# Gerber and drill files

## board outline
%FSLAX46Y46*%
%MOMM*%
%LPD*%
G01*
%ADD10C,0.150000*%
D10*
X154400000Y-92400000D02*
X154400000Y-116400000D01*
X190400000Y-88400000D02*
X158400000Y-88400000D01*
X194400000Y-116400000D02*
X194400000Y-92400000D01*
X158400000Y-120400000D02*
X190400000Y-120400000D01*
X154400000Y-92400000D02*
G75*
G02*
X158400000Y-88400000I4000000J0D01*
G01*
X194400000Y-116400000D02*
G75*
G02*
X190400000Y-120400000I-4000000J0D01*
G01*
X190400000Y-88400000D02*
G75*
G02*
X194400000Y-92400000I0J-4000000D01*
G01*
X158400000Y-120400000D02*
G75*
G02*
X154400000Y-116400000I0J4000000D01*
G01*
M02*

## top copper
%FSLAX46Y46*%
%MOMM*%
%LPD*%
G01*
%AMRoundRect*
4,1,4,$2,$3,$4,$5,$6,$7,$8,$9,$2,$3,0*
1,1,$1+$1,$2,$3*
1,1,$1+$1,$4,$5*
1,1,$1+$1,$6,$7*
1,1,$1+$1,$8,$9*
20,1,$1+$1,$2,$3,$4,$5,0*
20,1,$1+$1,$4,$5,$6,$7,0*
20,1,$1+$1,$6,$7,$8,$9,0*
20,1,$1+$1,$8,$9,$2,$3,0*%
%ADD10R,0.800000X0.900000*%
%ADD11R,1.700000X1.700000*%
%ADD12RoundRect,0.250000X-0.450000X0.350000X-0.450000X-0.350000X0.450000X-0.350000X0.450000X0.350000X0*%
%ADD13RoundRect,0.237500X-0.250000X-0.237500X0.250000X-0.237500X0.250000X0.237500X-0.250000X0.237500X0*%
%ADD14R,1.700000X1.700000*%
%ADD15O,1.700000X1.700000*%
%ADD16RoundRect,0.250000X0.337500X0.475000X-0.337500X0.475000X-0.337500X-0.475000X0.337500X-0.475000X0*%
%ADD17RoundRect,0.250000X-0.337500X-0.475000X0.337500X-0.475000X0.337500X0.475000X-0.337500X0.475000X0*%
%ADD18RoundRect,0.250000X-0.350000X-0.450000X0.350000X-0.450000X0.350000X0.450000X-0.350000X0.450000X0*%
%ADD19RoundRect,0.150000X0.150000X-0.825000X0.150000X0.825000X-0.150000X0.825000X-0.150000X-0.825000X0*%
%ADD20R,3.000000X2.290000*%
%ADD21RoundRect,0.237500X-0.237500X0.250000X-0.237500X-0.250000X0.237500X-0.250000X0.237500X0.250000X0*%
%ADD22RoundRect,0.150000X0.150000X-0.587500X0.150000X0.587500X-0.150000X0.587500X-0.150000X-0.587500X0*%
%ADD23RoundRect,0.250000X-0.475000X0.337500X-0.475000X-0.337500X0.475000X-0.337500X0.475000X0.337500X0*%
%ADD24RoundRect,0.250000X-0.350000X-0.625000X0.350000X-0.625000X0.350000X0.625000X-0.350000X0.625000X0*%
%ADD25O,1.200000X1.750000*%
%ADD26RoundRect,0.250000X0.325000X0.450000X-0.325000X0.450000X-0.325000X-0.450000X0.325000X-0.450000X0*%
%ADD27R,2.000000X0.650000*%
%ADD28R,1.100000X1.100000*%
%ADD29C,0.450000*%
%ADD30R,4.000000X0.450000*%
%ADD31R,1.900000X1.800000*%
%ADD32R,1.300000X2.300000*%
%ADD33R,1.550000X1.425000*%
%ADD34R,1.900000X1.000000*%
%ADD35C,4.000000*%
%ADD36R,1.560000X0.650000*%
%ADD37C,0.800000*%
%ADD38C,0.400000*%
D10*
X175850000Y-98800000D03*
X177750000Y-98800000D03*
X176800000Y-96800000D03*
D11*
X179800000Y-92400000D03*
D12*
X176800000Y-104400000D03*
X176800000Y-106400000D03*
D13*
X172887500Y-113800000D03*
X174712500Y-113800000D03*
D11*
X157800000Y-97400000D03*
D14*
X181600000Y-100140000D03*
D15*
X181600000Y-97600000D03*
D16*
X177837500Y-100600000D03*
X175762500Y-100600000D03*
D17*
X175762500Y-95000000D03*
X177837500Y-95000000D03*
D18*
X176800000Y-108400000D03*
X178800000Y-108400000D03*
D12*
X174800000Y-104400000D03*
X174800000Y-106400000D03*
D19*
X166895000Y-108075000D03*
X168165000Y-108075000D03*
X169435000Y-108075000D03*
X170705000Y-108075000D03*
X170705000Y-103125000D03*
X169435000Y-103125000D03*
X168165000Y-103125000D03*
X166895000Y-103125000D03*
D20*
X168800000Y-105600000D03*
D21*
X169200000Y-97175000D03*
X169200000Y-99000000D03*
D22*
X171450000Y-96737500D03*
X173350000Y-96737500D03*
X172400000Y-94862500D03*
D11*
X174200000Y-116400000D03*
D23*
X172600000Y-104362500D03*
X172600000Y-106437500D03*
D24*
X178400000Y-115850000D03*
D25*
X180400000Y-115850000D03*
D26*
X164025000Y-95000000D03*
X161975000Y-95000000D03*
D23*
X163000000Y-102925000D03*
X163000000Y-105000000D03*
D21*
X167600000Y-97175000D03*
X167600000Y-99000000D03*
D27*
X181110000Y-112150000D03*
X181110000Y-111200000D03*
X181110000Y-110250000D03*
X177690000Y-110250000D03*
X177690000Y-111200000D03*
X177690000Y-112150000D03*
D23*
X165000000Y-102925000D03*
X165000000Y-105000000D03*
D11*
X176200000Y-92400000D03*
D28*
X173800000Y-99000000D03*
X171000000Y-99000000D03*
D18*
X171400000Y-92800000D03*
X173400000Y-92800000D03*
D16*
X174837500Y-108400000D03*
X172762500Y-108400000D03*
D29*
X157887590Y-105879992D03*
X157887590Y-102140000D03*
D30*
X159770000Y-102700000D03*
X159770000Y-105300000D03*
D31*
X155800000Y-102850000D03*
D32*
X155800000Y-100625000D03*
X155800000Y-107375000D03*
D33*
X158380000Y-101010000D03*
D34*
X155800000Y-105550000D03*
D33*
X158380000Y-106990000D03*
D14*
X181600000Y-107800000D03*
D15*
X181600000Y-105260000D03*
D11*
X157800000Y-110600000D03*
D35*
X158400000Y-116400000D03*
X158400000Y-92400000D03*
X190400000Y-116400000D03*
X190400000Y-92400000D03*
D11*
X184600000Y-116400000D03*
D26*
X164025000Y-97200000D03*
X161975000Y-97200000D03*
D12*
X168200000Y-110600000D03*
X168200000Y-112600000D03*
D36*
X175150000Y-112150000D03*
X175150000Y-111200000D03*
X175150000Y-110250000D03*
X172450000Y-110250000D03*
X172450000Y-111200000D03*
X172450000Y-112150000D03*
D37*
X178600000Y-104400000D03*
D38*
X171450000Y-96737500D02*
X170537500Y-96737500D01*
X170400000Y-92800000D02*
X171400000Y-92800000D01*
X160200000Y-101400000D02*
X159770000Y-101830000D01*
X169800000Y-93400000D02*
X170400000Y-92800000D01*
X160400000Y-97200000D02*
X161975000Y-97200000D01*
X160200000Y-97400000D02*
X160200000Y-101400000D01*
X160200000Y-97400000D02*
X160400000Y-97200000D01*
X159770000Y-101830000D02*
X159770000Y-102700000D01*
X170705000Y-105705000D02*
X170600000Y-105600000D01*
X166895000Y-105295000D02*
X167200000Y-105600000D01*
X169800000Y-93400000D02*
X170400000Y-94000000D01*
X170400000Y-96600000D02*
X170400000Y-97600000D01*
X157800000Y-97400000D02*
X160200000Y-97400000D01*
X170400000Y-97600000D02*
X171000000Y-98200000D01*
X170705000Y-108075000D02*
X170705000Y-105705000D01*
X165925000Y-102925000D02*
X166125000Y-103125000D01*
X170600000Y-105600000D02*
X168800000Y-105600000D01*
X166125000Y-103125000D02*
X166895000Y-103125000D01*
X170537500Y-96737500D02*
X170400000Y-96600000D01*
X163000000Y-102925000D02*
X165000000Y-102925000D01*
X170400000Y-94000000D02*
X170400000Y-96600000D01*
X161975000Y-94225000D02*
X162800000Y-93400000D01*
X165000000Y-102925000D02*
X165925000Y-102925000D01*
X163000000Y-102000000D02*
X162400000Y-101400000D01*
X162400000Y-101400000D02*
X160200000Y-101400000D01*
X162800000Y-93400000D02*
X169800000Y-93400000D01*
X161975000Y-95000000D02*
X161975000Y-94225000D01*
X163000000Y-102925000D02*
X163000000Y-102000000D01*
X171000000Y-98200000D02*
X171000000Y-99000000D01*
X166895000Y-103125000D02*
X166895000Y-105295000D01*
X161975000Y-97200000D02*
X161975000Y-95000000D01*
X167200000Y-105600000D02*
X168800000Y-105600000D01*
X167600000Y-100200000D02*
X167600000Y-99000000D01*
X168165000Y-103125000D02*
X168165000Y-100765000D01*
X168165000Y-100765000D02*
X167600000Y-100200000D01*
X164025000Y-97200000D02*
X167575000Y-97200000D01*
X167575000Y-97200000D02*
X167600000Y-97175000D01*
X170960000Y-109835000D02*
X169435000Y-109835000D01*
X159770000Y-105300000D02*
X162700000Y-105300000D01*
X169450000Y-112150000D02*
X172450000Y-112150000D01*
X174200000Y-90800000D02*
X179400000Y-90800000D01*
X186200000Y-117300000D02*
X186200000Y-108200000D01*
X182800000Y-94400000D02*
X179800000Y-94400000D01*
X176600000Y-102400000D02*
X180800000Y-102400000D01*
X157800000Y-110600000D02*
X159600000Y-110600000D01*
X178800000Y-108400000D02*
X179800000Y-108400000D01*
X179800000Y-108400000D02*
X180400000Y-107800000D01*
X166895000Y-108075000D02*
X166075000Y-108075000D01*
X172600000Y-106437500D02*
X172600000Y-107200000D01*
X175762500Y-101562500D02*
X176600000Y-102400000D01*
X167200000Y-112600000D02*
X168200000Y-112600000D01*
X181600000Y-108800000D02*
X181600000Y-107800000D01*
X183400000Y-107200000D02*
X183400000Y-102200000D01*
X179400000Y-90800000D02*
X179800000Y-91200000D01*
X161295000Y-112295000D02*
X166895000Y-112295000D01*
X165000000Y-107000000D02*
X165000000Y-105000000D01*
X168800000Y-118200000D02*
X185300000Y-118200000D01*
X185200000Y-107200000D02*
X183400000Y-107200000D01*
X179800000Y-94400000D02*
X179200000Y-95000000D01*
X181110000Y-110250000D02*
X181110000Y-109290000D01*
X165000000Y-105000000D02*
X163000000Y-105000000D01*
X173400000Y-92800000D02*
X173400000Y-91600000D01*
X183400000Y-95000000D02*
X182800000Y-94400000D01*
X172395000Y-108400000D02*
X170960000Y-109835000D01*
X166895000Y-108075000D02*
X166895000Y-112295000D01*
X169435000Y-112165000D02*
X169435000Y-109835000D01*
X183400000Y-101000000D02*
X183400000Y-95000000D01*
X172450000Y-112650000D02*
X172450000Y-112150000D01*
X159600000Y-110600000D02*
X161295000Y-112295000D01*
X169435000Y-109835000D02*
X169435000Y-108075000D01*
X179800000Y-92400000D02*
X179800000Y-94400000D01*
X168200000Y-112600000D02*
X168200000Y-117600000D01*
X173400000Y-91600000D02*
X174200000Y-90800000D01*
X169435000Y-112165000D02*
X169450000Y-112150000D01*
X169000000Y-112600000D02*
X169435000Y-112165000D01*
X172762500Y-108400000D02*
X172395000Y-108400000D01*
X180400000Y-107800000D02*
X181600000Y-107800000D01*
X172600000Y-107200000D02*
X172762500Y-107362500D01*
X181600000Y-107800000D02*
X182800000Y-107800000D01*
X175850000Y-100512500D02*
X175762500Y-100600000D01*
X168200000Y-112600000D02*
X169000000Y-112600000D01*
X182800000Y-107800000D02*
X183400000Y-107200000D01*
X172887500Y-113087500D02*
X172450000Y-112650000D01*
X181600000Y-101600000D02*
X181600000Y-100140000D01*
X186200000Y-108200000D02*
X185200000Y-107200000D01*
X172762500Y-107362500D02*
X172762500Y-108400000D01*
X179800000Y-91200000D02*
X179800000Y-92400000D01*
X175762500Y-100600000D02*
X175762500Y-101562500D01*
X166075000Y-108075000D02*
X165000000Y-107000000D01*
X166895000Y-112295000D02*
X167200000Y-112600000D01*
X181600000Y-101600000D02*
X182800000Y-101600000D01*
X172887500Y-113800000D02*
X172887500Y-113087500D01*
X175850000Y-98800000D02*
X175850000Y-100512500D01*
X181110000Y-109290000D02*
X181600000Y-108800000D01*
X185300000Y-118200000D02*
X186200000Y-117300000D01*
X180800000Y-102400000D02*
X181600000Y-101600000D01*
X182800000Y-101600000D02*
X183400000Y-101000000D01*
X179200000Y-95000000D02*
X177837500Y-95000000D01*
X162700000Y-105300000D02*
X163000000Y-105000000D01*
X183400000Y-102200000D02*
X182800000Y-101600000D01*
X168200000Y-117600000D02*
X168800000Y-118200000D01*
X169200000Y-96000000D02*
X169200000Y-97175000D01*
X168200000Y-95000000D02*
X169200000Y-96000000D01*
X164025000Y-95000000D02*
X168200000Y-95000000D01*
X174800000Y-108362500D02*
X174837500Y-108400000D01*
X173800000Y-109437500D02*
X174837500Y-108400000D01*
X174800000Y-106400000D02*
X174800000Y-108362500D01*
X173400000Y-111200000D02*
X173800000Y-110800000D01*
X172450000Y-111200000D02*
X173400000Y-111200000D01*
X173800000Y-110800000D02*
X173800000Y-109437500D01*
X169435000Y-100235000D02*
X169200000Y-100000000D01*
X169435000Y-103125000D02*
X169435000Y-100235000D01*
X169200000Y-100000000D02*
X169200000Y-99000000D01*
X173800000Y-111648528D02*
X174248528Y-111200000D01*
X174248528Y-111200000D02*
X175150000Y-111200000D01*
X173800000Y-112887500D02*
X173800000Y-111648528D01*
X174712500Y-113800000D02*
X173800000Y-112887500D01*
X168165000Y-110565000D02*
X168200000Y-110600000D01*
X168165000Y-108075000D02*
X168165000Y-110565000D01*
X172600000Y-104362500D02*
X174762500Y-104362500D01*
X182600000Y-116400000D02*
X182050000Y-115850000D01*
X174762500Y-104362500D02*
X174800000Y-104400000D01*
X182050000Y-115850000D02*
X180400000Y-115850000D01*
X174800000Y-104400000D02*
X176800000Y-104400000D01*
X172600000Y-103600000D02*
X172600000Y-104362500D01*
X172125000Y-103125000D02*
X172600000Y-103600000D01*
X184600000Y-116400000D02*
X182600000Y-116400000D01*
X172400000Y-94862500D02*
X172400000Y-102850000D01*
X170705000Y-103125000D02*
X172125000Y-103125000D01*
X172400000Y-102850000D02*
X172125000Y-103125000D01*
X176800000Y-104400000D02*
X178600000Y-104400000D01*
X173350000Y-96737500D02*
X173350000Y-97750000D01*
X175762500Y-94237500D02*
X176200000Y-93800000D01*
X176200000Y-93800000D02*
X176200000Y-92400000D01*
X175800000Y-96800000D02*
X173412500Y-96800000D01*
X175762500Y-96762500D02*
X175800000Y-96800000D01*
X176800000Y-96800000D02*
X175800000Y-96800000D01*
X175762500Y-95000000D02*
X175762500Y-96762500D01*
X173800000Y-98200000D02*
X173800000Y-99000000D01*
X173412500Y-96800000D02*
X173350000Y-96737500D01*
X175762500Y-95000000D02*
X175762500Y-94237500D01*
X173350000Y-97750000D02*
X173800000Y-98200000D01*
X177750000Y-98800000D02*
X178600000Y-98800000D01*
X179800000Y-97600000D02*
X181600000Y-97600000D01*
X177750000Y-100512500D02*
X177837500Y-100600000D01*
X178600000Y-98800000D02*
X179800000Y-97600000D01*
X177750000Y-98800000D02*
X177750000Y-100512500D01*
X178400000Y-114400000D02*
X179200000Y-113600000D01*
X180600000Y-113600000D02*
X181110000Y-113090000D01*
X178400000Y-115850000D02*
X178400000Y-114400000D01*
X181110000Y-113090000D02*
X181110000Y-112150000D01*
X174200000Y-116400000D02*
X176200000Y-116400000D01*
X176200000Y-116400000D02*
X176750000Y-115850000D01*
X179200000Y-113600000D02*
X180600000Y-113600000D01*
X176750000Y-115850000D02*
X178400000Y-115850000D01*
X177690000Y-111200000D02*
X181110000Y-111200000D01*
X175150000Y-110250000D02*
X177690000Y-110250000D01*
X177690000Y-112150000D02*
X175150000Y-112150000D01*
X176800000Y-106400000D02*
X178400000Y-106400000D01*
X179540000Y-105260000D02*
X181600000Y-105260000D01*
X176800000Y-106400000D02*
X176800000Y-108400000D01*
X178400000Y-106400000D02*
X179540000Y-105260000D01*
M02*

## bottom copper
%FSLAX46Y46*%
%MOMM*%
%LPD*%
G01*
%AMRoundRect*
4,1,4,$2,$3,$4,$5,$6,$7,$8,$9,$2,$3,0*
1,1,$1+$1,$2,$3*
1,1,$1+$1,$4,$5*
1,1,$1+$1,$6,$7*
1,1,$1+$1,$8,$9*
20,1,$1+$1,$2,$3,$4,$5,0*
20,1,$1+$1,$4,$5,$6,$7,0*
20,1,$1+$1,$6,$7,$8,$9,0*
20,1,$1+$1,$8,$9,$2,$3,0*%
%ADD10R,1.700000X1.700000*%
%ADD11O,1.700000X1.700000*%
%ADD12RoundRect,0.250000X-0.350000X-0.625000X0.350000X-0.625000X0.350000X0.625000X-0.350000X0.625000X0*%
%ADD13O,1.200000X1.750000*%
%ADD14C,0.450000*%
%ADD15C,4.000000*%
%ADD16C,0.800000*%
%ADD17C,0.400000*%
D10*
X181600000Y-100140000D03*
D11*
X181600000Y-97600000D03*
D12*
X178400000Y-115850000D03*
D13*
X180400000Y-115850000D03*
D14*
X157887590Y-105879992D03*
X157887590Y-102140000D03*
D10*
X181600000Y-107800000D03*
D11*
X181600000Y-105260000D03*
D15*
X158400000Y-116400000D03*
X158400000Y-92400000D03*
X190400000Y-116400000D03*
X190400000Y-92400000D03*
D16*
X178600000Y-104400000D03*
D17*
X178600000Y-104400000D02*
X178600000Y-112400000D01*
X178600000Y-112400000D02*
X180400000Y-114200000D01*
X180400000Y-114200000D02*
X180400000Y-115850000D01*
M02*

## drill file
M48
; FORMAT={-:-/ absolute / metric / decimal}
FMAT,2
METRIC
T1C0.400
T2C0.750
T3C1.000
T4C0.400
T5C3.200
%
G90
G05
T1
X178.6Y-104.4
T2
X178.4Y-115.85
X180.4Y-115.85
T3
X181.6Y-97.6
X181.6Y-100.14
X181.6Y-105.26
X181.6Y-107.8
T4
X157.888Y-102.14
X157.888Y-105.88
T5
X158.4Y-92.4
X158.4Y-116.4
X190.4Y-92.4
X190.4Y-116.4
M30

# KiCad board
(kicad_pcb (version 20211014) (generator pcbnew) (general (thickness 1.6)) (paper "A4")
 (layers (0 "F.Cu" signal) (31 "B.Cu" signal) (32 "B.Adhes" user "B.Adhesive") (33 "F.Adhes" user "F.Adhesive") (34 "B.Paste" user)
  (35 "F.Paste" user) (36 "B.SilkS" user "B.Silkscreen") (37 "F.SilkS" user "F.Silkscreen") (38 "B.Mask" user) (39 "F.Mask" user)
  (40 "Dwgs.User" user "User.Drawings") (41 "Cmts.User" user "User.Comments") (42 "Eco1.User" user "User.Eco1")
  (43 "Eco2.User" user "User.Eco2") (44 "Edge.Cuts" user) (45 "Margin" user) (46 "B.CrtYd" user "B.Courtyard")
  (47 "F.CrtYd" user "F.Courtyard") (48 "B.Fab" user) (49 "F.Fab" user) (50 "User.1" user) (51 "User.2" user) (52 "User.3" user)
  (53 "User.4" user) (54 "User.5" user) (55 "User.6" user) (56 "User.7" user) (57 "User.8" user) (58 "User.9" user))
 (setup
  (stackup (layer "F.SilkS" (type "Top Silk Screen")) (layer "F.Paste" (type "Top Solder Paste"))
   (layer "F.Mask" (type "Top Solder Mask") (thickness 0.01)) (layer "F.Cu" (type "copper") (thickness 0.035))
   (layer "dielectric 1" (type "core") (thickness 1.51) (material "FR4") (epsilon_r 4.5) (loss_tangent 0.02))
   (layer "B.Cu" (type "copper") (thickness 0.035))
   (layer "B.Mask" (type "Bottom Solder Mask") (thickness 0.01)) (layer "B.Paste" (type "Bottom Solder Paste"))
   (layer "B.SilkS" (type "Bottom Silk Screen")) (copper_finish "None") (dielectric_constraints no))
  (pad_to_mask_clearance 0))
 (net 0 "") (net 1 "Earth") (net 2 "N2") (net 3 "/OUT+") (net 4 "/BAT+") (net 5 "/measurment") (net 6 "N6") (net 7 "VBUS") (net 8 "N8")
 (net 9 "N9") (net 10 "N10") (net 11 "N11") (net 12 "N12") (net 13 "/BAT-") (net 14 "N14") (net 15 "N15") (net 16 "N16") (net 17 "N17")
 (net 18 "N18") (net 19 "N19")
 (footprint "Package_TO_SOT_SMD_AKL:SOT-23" (layer "F.Cu") (at 176.8 97.8 90)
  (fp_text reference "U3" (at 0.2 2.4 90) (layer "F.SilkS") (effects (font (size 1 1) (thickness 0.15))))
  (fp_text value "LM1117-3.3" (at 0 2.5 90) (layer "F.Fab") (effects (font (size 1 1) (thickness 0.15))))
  (pad "1" smd rect (at -1 -0.95 90) (size 0.9 0.8) (layers "F.Cu" "F.Paste" "F.Mask") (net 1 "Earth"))
  (pad "2" smd rect (at -1 0.95 90) (size 0.9 0.8) (layers "F.Cu" "F.Paste" "F.Mask") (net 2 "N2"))
  (pad "3" smd rect (at 1 0 90) (size 0.9 0.8) (layers "F.Cu" "F.Paste" "F.Mask") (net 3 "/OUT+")))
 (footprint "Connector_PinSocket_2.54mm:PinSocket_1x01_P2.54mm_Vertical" (layer "F.Cu") (at 179.8 92.4)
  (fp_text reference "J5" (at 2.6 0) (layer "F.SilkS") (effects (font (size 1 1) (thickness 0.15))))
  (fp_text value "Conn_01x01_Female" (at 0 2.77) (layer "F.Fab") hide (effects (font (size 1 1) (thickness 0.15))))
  (pad "1" smd rect (at 0 0) (size 1.7 1.7) (layers "F.Cu" "F.Paste" "F.Mask") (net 1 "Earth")))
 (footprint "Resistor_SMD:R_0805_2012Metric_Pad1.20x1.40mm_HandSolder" (layer "F.Cu") (at 176.8 105.4 -90)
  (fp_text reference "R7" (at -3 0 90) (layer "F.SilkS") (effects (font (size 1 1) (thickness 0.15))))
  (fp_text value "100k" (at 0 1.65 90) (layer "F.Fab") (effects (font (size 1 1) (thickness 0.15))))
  (pad "1" smd roundrect (at -1 0 270) (size 1.2 1.4) (layers "F.Cu" "F.Paste" "F.Mask") (roundrect_rratio 0.208333) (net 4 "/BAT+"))
  (pad "2" smd roundrect (at 1 0 270) (size 1.2 1.4) (layers "F.Cu" "F.Paste" "F.Mask") (roundrect_rratio 0.208333) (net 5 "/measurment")))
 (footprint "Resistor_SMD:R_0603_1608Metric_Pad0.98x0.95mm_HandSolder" (layer "F.Cu") (at 173.8 113.8)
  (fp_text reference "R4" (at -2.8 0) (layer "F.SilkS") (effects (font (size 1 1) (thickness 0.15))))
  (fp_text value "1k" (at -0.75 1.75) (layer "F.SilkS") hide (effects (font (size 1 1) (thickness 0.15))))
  (pad "1" smd roundrect (at -0.9125 0) (size 0.975 0.95) (layers "F.Cu" "F.Paste" "F.Mask") (roundrect_rratio 0.25) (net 1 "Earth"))
  (pad "2" smd roundrect (at 0.9125 0) (size 0.975 0.95) (layers "F.Cu" "F.Paste" "F.Mask") (roundrect_rratio 0.25) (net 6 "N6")))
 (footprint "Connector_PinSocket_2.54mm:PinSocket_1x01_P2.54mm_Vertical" (layer "F.Cu") (at 157.8 97.4)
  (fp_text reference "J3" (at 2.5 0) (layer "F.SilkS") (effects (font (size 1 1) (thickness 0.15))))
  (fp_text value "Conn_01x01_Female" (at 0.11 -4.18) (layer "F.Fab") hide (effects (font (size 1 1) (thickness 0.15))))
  (pad "1" smd rect (at 0 0) (size 1.7 1.7) (layers "F.Cu" "F.Paste" "F.Mask") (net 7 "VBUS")))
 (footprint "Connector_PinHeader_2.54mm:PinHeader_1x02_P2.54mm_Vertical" (layer "F.Cu") (at 181.6 100.14 180)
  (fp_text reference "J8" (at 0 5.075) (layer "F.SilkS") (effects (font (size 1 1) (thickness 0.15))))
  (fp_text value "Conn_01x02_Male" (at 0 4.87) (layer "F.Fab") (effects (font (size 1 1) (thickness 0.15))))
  (pad "1" thru_hole rect (at 0 0 180) (size 1.7 1.7) (drill 1) (layers *.Cu *.Mask) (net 1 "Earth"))
  (pad "2" thru_hole oval (at 0 2.54 180) (size 1.7 1.7) (drill 1) (layers *.Cu *.Mask) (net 2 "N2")))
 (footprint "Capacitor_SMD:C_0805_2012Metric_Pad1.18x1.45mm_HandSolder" (layer "F.Cu") (at 176.8 100.6 180)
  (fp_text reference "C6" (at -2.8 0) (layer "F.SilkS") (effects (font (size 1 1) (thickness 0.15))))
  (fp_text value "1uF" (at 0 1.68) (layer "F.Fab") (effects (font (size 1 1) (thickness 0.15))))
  (pad "1" smd roundrect (at -1.0375 0 180) (size 1.175 1.45) (layers "F.Cu" "F.Paste" "F.Mask") (roundrect_rratio 0.212766) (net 2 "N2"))
  (pad "2" smd roundrect (at 1.0375 0 180) (size 1.175 1.45) (layers "F.Cu" "F.Paste" "F.Mask") (roundrect_rratio 0.212766) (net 1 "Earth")))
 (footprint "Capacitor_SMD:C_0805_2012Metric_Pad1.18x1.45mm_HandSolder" (layer "F.Cu") (at 176.8 95)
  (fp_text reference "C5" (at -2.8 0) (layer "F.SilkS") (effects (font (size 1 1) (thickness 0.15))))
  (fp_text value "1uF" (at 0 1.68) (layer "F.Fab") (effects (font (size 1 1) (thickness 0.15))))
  (pad "1" smd roundrect (at -1.0375 0) (size 1.175 1.45) (layers "F.Cu" "F.Paste" "F.Mask") (roundrect_rratio 0.212766) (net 3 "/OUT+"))
  (pad "2" smd roundrect (at 1.0375 0) (size 1.175 1.45) (layers "F.Cu" "F.Paste" "F.Mask") (roundrect_rratio 0.212766) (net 1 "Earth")))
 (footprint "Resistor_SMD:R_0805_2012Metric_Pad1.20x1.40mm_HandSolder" (layer "F.Cu") (at 177.8 108.4)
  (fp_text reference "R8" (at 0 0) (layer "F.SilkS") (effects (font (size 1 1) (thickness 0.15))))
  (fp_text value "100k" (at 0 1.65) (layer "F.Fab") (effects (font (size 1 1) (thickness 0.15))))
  (pad "1" smd roundrect (at -1 0) (size 1.2 1.4) (layers "F.Cu" "F.Paste" "F.Mask") (roundrect_rratio 0.208333) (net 5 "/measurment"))
  (pad "2" smd roundrect (at 1 0) (size 1.2 1.4) (layers "F.Cu" "F.Paste" "F.Mask") (roundrect_rratio 0.208333) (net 1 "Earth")))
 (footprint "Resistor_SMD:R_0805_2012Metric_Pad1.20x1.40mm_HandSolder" (layer "F.Cu") (at 174.8 105.4 -90)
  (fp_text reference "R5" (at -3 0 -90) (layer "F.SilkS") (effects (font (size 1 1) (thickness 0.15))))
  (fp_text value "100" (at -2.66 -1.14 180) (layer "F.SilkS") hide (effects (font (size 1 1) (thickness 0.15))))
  (pad "1" smd roundrect (at -1 0 270) (size 1.2 1.4) (layers "F.Cu" "F.Paste" "F.Mask") (roundrect_rratio 0.2083333333) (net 4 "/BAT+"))
  (pad "2" smd roundrect (at 1 0 270) (size 1.2 1.4) (layers "F.Cu" "F.Paste" "F.Mask") (roundrect_rratio 0.2083333333) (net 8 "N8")))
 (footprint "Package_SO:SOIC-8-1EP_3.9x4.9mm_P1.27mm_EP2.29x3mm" (layer "F.Cu") (at 168.8 105.6 90)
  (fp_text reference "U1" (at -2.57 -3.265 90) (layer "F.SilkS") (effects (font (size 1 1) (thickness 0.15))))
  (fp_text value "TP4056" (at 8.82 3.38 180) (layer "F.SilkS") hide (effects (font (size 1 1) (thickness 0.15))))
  (pad "" smd roundrect (at 0.57 0.75 90) (size 0.92 1.21) (layers "F.Paste") (roundrect_rratio 0.25))
  (pad "" smd roundrect (at 0.57 -0.75 90) (size 0.92 1.21) (layers "F.Paste") (roundrect_rratio 0.25))
  (pad "" smd roundrect (at -0.57 0.75 90) (size 0.92 1.21) (layers "F.Paste") (roundrect_rratio 0.25))
  (pad "" smd roundrect (at -0.57 -0.75 90) (size 0.92 1.21) (layers "F.Paste") (roundrect_rratio 0.25))
  (pad "1" smd roundrect (at -2.475 -1.905 90) (size 1.95 0.6) (layers "F.Cu" "F.Paste" "F.Mask") (roundrect_rratio 0.25) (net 1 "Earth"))
  (pad "2" smd roundrect (at -2.475 -0.635 90) (size 1.95 0.6) (layers "F.Cu" "F.Paste" "F.Mask") (roundrect_rratio 0.25) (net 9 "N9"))
  (pad "3" smd roundrect (at -2.475 0.635 90) (size 1.95 0.6) (layers "F.Cu" "F.Paste" "F.Mask") (roundrect_rratio 0.25) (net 1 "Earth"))
  (pad "4" smd roundrect (at -2.475 1.905 90) (size 1.95 0.6) (layers "F.Cu" "F.Paste" "F.Mask") (roundrect_rratio 0.25) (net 7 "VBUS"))
  (pad "5" smd roundrect (at 2.475 1.905 90) (size 1.95 0.6) (layers "F.Cu" "F.Paste" "F.Mask") (roundrect_rratio 0.25) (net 4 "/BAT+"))
  (pad "6" smd roundrect (at 2.475 0.635 90) (size 1.95 0.6) (layers "F.Cu" "F.Paste" "F.Mask") (roundrect_rratio 0.25) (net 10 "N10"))
  (pad "7" smd roundrect (at 2.475 -0.635 90) (size 1.95 0.6) (layers "F.Cu" "F.Paste" "F.Mask") (roundrect_rratio 0.25) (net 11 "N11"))
  (pad "8" smd roundrect (at 2.475 -1.905 90) (size 1.95 0.6) (layers "F.Cu" "F.Paste" "F.Mask") (roundrect_rratio 0.25) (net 7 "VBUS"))
  (pad "9" smd rect (at 0 0 90) (size 2.29 3) (layers "F.Cu" "F.Mask") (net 7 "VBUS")))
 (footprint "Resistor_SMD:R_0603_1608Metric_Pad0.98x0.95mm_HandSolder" (layer "F.Cu") (at 169.2 98.0875 -90)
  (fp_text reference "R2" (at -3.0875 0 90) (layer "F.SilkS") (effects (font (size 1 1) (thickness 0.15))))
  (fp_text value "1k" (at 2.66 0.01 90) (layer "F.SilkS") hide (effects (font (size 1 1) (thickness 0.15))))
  (pad "1" smd roundrect (at -0.9125 0 270) (size 0.975 0.95) (layers "F.Cu" "F.Paste" "F.Mask") (roundrect_rratio 0.25) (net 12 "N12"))
  (pad "2" smd roundrect (at 0.9125 0 270) (size 0.975 0.95) (layers "F.Cu" "F.Paste" "F.Mask") (roundrect_rratio 0.25) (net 10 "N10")))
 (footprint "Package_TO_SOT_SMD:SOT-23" (layer "F.Cu") (at 172.4 95.8 90)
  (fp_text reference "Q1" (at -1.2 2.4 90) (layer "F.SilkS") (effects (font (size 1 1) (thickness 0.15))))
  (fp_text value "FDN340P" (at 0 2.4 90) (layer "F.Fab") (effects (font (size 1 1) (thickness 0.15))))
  (pad "1" smd roundrect (at -0.9375 -0.95 90) (size 1.475 0.6) (layers "F.Cu" "F.Paste" "F.Mask") (roundrect_rratio 0.25) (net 7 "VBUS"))
  (pad "2" smd roundrect (at -0.9375 0.95 90) (size 1.475 0.6) (layers "F.Cu" "F.Paste" "F.Mask") (roundrect_rratio 0.25) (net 3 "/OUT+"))
  (pad "3" smd roundrect (at 0.9375 0 90) (size 1.475 0.6) (layers "F.Cu" "F.Paste" "F.Mask") (roundrect_rratio 0.25) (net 4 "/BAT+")))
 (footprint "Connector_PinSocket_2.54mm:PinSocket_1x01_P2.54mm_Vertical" (layer "F.Cu") (at 174.2 116.4)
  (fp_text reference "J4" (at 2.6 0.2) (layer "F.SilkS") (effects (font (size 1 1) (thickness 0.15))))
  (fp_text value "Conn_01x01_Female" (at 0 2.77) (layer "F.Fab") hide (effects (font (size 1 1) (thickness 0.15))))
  (pad "1" smd rect (at 0 0) (size 1.7 1.7) (layers "F.Cu" "F.Paste" "F.Mask") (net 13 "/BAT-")))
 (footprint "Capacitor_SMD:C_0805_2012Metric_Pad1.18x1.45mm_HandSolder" (layer "F.Cu") (at 172.6 105.4 -90)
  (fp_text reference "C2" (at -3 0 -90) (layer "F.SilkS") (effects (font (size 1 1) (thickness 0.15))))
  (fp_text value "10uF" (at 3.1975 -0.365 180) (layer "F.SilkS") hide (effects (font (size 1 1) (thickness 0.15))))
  (pad "1" smd roundrect (at -1.0375 0 270) (size 1.175 1.45) (layers "F.Cu" "F.Paste" "F.Mask") (roundrect_rratio 0.2127659574)
   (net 4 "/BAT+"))
  (pad "2" smd roundrect (at 1.0375 0 270) (size 1.175 1.45) (layers "F.Cu" "F.Paste" "F.Mask") (roundrect_rratio 0.2127659574)
   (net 1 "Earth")))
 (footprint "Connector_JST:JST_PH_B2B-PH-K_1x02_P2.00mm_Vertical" (layer "F.Cu") (at 178.4 115.85)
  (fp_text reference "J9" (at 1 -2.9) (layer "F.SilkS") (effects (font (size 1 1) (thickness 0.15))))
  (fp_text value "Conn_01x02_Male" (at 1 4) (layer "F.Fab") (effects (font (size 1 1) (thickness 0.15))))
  (pad "1" thru_hole roundrect (at 0 0) (size 1.2 1.75) (drill 0.75) (layers *.Cu *.Mask) (roundrect_rratio 0.208333) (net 13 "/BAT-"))
  (pad "2" thru_hole oval (at 2 0) (size 1.2 1.75) (drill 0.75) (layers *.Cu *.Mask) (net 4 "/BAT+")))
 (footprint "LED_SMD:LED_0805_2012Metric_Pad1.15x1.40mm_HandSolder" (layer "F.Cu") (at 163 95 180)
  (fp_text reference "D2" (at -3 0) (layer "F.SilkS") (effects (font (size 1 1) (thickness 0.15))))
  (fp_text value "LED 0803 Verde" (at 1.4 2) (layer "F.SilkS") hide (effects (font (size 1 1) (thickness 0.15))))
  (pad "1" smd roundrect (at -1.025 0 180) (size 1.15 1.4) (layers "F.Cu" "F.Paste" "F.Mask") (roundrect_rratio 0.2173913043) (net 12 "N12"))
  (pad "2" smd roundrect (at 1.025 0 180) (size 1.15 1.4) (layers "F.Cu" "F.Paste" "F.Mask") (roundrect_rratio 0.2173913043) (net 7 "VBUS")))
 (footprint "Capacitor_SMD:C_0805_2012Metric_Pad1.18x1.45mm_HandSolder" (layer "F.Cu") (at 163 103.9625 -90)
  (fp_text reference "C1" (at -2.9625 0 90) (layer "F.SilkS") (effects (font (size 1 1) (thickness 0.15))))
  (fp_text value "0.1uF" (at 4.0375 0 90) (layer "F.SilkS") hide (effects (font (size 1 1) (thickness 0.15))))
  (pad "1" smd roundrect (at -1.0375 0 270) (size 1.175 1.45) (layers "F.Cu" "F.Paste" "F.Mask") (roundrect_rratio 0.2127659574)
   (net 7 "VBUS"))
  (pad "2" smd roundrect (at 1.0375 0 270) (size 1.175 1.45) (layers "F.Cu" "F.Paste" "F.Mask") (roundrect_rratio 0.2127659574)
   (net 1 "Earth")))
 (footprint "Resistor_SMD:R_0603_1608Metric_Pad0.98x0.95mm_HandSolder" (layer "F.Cu") (at 167.6 98.0875 -90)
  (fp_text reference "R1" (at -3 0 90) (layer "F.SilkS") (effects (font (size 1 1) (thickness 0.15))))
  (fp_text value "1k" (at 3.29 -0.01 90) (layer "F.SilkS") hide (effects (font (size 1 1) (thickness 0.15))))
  (pad "1" smd roundrect (at -0.9125 0 270) (size 0.975 0.95) (layers "F.Cu" "F.Paste" "F.Mask") (roundrect_rratio 0.25) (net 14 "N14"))
  (pad "2" smd roundrect (at 0.9125 0 270) (size 0.975 0.95) (layers "F.Cu" "F.Paste" "F.Mask") (roundrect_rratio 0.25) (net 11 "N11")))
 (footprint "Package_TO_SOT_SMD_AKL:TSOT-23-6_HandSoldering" (layer "F.Cu") (at 179.4 111.2 180)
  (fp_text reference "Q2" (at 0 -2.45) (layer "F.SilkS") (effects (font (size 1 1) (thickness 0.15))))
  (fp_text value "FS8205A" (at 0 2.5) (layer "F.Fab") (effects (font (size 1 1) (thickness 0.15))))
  (pad "1" smd rect (at -1.71 -0.95 180) (size 2 0.65) (layers "F.Cu" "F.Paste" "F.Mask") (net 13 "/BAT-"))
  (pad "2" smd rect (at -1.71 0 180) (size 2 0.65) (layers "F.Cu" "F.Paste" "F.Mask") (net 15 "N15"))
  (pad "3" smd rect (at -1.71 0.95 180) (size 2 0.65) (layers "F.Cu" "F.Paste" "F.Mask") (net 1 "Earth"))
  (pad "4" smd rect (at 1.71 0.95 180) (size 2 0.65) (layers "F.Cu" "F.Paste" "F.Mask") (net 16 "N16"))
  (pad "5" smd rect (at 1.71 0 180) (size 2 0.65) (layers "F.Cu" "F.Paste" "F.Mask") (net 15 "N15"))
  (pad "6" smd rect (at 1.71 -0.95 180) (size 2 0.65) (layers "F.Cu" "F.Paste" "F.Mask") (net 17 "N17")))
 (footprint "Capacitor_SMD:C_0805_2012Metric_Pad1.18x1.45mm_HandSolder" (layer "F.Cu") (at 165 103.9625 -90)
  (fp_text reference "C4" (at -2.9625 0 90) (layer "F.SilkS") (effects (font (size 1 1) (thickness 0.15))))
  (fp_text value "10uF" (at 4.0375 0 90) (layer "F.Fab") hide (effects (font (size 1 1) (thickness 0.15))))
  (pad "1" smd roundrect (at -1.0375 0 270) (size 1.175 1.45) (layers "F.Cu" "F.Paste" "F.Mask") (roundrect_rratio 0.212766) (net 7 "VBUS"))
  (pad "2" smd roundrect (at 1.0375 0 270) (size 1.175 1.45) (layers "F.Cu" "F.Paste" "F.Mask") (roundrect_rratio 0.212766) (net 1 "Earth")))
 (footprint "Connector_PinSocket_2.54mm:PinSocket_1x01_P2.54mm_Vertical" (layer "F.Cu") (at 176.2 92.4)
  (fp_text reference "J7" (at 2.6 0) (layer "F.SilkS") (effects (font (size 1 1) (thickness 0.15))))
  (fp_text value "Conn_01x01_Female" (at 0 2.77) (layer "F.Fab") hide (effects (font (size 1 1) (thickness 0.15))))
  (pad "1" smd rect (at 0 0) (size 1.7 1.7) (layers "F.Cu" "F.Paste" "F.Mask") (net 3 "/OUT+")))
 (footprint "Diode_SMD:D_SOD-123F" (layer "F.Cu") (at 172.4 99 180)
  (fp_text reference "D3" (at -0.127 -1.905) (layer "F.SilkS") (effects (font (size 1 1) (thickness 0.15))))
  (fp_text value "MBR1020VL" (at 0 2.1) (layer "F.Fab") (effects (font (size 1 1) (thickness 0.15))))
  (pad "1" smd rect (at -1.4 0 180) (size 1.1 1.1) (layers "F.Cu" "F.Paste" "F.Mask") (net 3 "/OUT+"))
  (pad "2" smd rect (at 1.4 0 180) (size 1.1 1.1) (layers "F.Cu" "F.Paste" "F.Mask") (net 7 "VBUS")))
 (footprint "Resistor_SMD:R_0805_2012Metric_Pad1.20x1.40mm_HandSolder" (layer "F.Cu") (at 172.4 92.8)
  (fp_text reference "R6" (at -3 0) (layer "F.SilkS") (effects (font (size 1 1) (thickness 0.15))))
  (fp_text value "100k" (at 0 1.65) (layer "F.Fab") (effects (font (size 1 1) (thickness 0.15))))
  (pad "1" smd roundrect (at -1 0) (size 1.2 1.4) (layers "F.Cu" "F.Paste" "F.Mask") (roundrect_rratio 0.208333) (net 7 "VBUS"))
  (pad "2" smd roundrect (at 1 0) (size 1.2 1.4) (layers "F.Cu" "F.Paste" "F.Mask") (roundrect_rratio 0.208333) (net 1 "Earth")))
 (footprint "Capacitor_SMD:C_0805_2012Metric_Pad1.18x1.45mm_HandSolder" (layer "F.Cu") (at 173.8 108.4 180)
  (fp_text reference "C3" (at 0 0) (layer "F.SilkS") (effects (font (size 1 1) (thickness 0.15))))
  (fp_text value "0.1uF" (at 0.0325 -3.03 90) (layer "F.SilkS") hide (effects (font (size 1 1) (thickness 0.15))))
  (pad "1" smd roundrect (at -1.0375 0 180) (size 1.175 1.45) (layers "F.Cu" "F.Paste" "F.Mask") (roundrect_rratio 0.2127659574)
   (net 8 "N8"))
  (pad "2" smd roundrect (at 1.0375 0 180) (size 1.175 1.45) (layers "F.Cu" "F.Paste" "F.Mask") (roundrect_rratio 0.2127659574)
   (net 1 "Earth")))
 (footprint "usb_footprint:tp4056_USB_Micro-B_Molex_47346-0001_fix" (layer "F.Cu") (at 157 104 -90)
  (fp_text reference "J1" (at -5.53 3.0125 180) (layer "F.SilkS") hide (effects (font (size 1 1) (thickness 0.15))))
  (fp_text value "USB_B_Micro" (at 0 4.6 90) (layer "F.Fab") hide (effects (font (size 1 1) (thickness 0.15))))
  (pad "" np_thru_hole circle (at 1.879992 -0.88759 270) (size 0.45 0.45) (drill 0.4) (layers F&B.Cu *.Mask) (clearance 0.02))
  (pad "" np_thru_hole circle (at -1.86 -0.88759 270) (size 0.45 0.45) (drill 0.4) (layers F&B.Cu *.Mask) (clearance 0.02))
  (pad "1" smd rect (at -1.3 -2.77 270) (size 0.45 4) (layers "F.Cu" "F.Paste" "F.Mask") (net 7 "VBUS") (clearance 0.02))
  (pad "5" smd rect (at 1.3 -2.77 270) (size 0.45 4) (layers "F.Cu" "F.Paste" "F.Mask") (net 1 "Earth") (clearance 0.02))
  (pad "6" smd rect (at -1.15 1.2 270) (size 1.8 1.9) (layers "F.Cu" "F.Paste" "F.Mask") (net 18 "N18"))
  (pad "6" smd rect (at -3.375 1.2 270) (size 2.3 1.3) (layers "F.Cu" "F.Paste" "F.Mask") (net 18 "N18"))
  (pad "6" smd rect (at 3.375 1.2 270) (size 2.3 1.3) (layers "F.Cu" "F.Paste" "F.Mask") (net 18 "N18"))
  (pad "6" smd rect (at -2.99 -1.38 270) (size 1.425 1.55) (layers "F.Cu" "F.Paste" "F.Mask") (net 18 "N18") (clearance 0.02))
  (pad "6" smd rect (at 1.55 1.2 270) (size 1 1.9) (layers "F.Cu" "F.Paste" "F.Mask") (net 18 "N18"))
  (pad "6" smd rect (at 2.99 -1.38 270) (size 1.425 1.55) (layers "F.Cu" "F.Paste" "F.Mask") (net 18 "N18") (clearance 0.02)))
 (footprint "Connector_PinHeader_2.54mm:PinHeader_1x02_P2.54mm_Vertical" (layer "F.Cu") (at 181.6 107.8 180)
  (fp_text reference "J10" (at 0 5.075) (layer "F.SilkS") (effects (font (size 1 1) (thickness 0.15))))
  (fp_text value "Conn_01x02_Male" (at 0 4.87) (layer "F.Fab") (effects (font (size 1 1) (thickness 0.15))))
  (pad "1" thru_hole rect (at 0 0 180) (size 1.7 1.7) (drill 1) (layers *.Cu *.Mask) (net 1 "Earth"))
  (pad "2" thru_hole oval (at 0 2.54 180) (size 1.7 1.7) (drill 1) (layers *.Cu *.Mask) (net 5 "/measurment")))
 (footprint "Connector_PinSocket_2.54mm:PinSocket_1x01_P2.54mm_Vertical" (layer "F.Cu") (at 157.8 110.6)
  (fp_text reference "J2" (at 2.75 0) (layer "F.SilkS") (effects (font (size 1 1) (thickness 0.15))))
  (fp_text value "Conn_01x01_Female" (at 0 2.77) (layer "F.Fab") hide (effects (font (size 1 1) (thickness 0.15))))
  (pad "1" smd rect (at 0 0) (size 1.7 1.7) (layers "F.Cu" "F.Paste" "F.Mask") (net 1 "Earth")))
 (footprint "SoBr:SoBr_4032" (layer "F.Cu") (at 154.4 120.4)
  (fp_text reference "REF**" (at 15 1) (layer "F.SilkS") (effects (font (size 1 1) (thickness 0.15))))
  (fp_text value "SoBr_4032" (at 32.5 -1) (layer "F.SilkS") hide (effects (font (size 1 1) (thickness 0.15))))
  (fp_line (start 0 -28) (end 0 -4) (layer "Edge.Cuts") (width 0.15))
  (fp_line (start 36 -32) (end 4 -32) (layer "Edge.Cuts") (width 0.15))
  (fp_line (start 40 -4) (end 40 -28) (layer "Edge.Cuts") (width 0.15))
  (fp_line (start 4 0) (end 36 0) (layer "Edge.Cuts") (width 0.15))
  (fp_arc (start 0 -28) (mid 1.171573 -30.828427) (end 4 -32) (layer "Edge.Cuts") (width 0.15))
  (fp_arc (start 40 -4) (mid 38.828427 -1.171573) (end 36 0) (layer "Edge.Cuts") (width 0.15))
  (fp_arc (start 36 -32) (mid 38.828427 -30.828427) (end 40 -28) (layer "Edge.Cuts") (width 0.15))
  (fp_arc (start 4 0) (mid 1.171573 -1.171573) (end 0 -4) (layer "Edge.Cuts") (width 0.15))
  (pad "" np_thru_hole circle locked (at 4 -4) (size 4 4) (drill 3.2) (layers *.Cu *.Mask))
  (pad "" np_thru_hole circle locked (at 4 -28) (size 4 4) (drill 3.2) (layers *.Cu *.Mask))
  (pad "" np_thru_hole circle locked (at 36 -4) (size 4 4) (drill 3.2) (layers *.Cu *.Mask))
  (pad "" np_thru_hole circle locked (at 36 -28) (size 4 4) (drill 3.2) (layers *.Cu *.Mask)))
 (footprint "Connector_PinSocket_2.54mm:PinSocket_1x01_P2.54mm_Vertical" (layer "F.Cu") (at 184.6 116.4)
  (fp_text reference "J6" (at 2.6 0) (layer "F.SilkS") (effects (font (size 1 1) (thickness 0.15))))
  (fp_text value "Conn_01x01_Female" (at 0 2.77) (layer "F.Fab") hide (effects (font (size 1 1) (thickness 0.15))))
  (pad "1" smd rect (at 0 0) (size 1.7 1.7) (layers "F.Cu" "F.Paste" "F.Mask") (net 4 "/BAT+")))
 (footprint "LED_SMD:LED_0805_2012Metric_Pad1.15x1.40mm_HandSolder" (layer "F.Cu") (at 163 97.2 180)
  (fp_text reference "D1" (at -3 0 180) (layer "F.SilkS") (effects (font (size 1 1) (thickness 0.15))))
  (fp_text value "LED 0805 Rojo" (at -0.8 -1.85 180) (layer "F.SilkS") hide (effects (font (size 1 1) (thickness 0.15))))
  (pad "1" smd roundrect (at -1.025 0 180) (size 1.15 1.4) (layers "F.Cu" "F.Paste" "F.Mask") (roundrect_rratio 0.2173913043) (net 14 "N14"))
  (pad "2" smd roundrect (at 1.025 0 180) (size 1.15 1.4) (layers "F.Cu" "F.Paste" "F.Mask") (roundrect_rratio 0.2173913043) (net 7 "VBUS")))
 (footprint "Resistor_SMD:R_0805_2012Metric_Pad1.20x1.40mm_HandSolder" (layer "F.Cu") (at 168.2 111.6 -90)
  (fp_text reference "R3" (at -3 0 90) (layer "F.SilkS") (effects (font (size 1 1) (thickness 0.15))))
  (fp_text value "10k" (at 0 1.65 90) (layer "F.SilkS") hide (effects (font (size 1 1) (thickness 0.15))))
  (pad "1" smd roundrect (at -1 0 270) (size 1.2 1.4) (layers "F.Cu" "F.Paste" "F.Mask") (roundrect_rratio 0.2083333333) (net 9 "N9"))
  (pad "2" smd roundrect (at 1 0 270) (size 1.2 1.4) (layers "F.Cu" "F.Paste" "F.Mask") (roundrect_rratio 0.2083333333) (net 1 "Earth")))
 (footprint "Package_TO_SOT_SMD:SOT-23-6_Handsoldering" (layer "F.Cu") (at 173.8 111.2 180)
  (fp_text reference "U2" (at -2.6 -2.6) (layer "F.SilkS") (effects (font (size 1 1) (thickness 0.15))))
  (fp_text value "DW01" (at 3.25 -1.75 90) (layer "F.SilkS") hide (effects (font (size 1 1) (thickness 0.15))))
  (pad "1" smd rect (at -1.35 -0.95 180) (size 1.56 0.65) (layers "F.Cu" "F.Paste" "F.Mask") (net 17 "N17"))
  (pad "2" smd rect (at -1.35 0 180) (size 1.56 0.65) (layers "F.Cu" "F.Paste" "F.Mask") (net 6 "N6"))
  (pad "3" smd rect (at -1.35 0.95 180) (size 1.56 0.65) (layers "F.Cu" "F.Paste" "F.Mask") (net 16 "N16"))
  (pad "4" smd rect (at 1.35 0.95 180) (size 1.56 0.65) (layers "F.Cu" "F.Paste" "F.Mask") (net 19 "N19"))
  (pad "5" smd rect (at 1.35 0 180) (size 1.56 0.65) (layers "F.Cu" "F.Paste" "F.Mask") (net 8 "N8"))
  (pad "6" smd rect (at 1.35 -0.95 180) (size 1.56 0.65) (layers "F.Cu" "F.Paste" "F.Mask") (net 1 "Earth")))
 (segment (start 171.45 96.7375) (end 170.5375 96.7375) (width 0.4) (layer "F.Cu") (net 7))
 (segment (start 170.4 92.8) (end 171.4 92.8) (width 0.4) (layer "F.Cu") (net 7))
 (segment (start 160.2 101.4) (end 159.77 101.83) (width 0.4) (layer "F.Cu") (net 7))
 (segment (start 169.8 93.4) (end 170.4 92.8) (width 0.4) (layer "F.Cu") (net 7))
 (segment (start 160.4 97.2) (end 161.975 97.2) (width 0.4) (layer "F.Cu") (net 7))
 (segment (start 160.2 97.4) (end 160.2 101.4) (width 0.4) (layer "F.Cu") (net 7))
 (segment (start 160.2 97.4) (end 160.4 97.2) (width 0.4) (layer "F.Cu") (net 7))
 (segment (start 159.77 101.83) (end 159.77 102.7) (width 0.4) (layer "F.Cu") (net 7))
 (segment (start 170.705 105.705) (end 170.6 105.6) (width 0.4) (layer "F.Cu") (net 7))
 (segment (start 166.895 105.295) (end 167.2 105.6) (width 0.4) (layer "F.Cu") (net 7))
 (segment (start 169.8 93.4) (end 170.4 94) (width 0.4) (layer "F.Cu") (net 7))
 (segment (start 170.4 96.6) (end 170.4 97.6) (width 0.4) (layer "F.Cu") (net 7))
 (segment (start 157.8 97.4) (end 160.2 97.4) (width 0.4) (layer "F.Cu") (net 7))
 (segment (start 170.4 97.6) (end 171 98.2) (width 0.4) (layer "F.Cu") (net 7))
 (segment (start 170.705 108.075) (end 170.705 105.705) (width 0.4) (layer "F.Cu") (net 7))
 (segment (start 165.925 102.925) (end 166.125 103.125) (width 0.4) (layer "F.Cu") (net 7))
 (segment (start 170.6 105.6) (end 168.8 105.6) (width 0.4) (layer "F.Cu") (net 7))
 (segment (start 166.125 103.125) (end 166.895 103.125) (width 0.4) (layer "F.Cu") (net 7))
 (segment (start 170.5375 96.7375) (end 170.4 96.6) (width 0.4) (layer "F.Cu") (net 7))
 (segment (start 163 102.925) (end 165 102.925) (width 0.4) (layer "F.Cu") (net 7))
 (segment (start 170.4 94) (end 170.4 96.6) (width 0.4) (layer "F.Cu") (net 7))
 (segment (start 161.975 94.225) (end 162.8 93.4) (width 0.4) (layer "F.Cu") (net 7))
 (segment (start 165 102.925) (end 165.925 102.925) (width 0.4) (layer "F.Cu") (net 7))
 (segment (start 163 102) (end 162.4 101.4) (width 0.4) (layer "F.Cu") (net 7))
 (segment (start 162.4 101.4) (end 160.2 101.4) (width 0.4) (layer "F.Cu") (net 7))
 (segment (start 162.8 93.4) (end 169.8 93.4) (width 0.4) (layer "F.Cu") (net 7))
 (segment (start 161.975 95) (end 161.975 94.225) (width 0.4) (layer "F.Cu") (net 7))
 (segment (start 163 102.925) (end 163 102) (width 0.4) (layer "F.Cu") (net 7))
 (segment (start 171 98.2) (end 171 99) (width 0.4) (layer "F.Cu") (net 7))
 (segment (start 166.895 103.125) (end 166.895 105.295) (width 0.4) (layer "F.Cu") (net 7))
 (segment (start 161.975 97.2) (end 161.975 95) (width 0.4) (layer "F.Cu") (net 7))
 (segment (start 167.2 105.6) (end 168.8 105.6) (width 0.4) (layer "F.Cu") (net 7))
 (segment (start 167.6 100.2) (end 167.6 99) (width 0.4) (layer "F.Cu") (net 11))
 (segment (start 168.165 103.125) (end 168.165 100.765) (width 0.4) (layer "F.Cu") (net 11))
 (segment (start 168.165 100.765) (end 167.6 100.2) (width 0.4) (layer "F.Cu") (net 11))
 (segment (start 164.025 97.2) (end 167.575 97.2) (width 0.4) (layer "F.Cu") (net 14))
 (segment (start 167.575 97.2) (end 167.6 97.175) (width 0.4) (layer "F.Cu") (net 14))
 (segment (start 170.96 109.835) (end 169.435 109.835) (width 0.4) (layer "F.Cu") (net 1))
 (segment (start 159.77 105.3) (end 162.7 105.3) (width 0.4) (layer "F.Cu") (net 1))
 (segment (start 169.45 112.15) (end 172.45 112.15) (width 0.4) (layer "F.Cu") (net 1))
 (segment (start 174.2 90.8) (end 179.4 90.8) (width 0.4) (layer "F.Cu") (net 1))
 (segment (start 186.2 117.3) (end 186.2 108.2) (width 0.4) (layer "F.Cu") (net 1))
 (segment (start 182.8 94.4) (end 179.8 94.4) (width 0.4) (layer "F.Cu") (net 1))
 (segment (start 176.6 102.4) (end 180.8 102.4) (width 0.4) (layer "F.Cu") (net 1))
 (segment (start 157.8 110.6) (end 159.6 110.6) (width 0.4) (layer "F.Cu") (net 1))
 (segment (start 178.8 108.4) (end 179.8 108.4) (width 0.4) (layer "F.Cu") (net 1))
 (segment (start 179.8 108.4) (end 180.4 107.8) (width 0.4) (layer "F.Cu") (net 1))
 (segment (start 166.895 108.075) (end 166.075 108.075) (width 0.4) (layer "F.Cu") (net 1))
 (segment (start 172.6 106.4375) (end 172.6 107.2) (width 0.4) (layer "F.Cu") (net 1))
 (segment (start 175.7625 101.5625) (end 176.6 102.4) (width 0.4) (layer "F.Cu") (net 1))
 (segment (start 167.2 112.6) (end 168.2 112.6) (width 0.4) (layer "F.Cu") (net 1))
 (segment (start 181.6 108.8) (end 181.6 107.8) (width 0.4) (layer "F.Cu") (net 1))
 (segment (start 183.4 107.2) (end 183.4 102.2) (width 0.4) (layer "F.Cu") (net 1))
 (segment (start 179.4 90.8) (end 179.8 91.2) (width 0.4) (layer "F.Cu") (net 1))
 (segment (start 161.295 112.295) (end 166.895 112.295) (width 0.4) (layer "F.Cu") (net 1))
 (segment (start 165 107) (end 165 105) (width 0.4) (layer "F.Cu") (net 1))
 (segment (start 168.8 118.2) (end 185.3 118.2) (width 0.4) (layer "F.Cu") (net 1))
 (segment (start 185.2 107.2) (end 183.4 107.2) (width 0.4) (layer "F.Cu") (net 1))
 (segment (start 179.8 94.4) (end 179.2 95) (width 0.4) (layer "F.Cu") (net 1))
 (segment (start 181.11 110.25) (end 181.11 109.29) (width 0.4) (layer "F.Cu") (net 1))
 (segment (start 165 105) (end 163 105) (width 0.4) (layer "F.Cu") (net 1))
 (segment (start 173.4 92.8) (end 173.4 91.6) (width 0.4) (layer "F.Cu") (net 1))
 (segment (start 183.4 95) (end 182.8 94.4) (width 0.4) (layer "F.Cu") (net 1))
 (segment (start 172.395 108.4) (end 170.96 109.835) (width 0.4) (layer "F.Cu") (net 1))
 (segment (start 166.895 108.075) (end 166.895 112.295) (width 0.4) (layer "F.Cu") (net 1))
 (segment (start 169.435 112.165) (end 169.435 109.835) (width 0.4) (layer "F.Cu") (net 1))
 (segment (start 183.4 101) (end 183.4 95) (width 0.4) (layer "F.Cu") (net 1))
 (segment (start 172.45 112.65) (end 172.45 112.15) (width 0.4) (layer "F.Cu") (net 1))
 (segment (start 159.6 110.6) (end 161.295 112.295) (width 0.4) (layer "F.Cu") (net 1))
 (segment (start 169.435 109.835) (end 169.435 108.075) (width 0.4) (layer "F.Cu") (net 1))
 (segment (start 179.8 92.4) (end 179.8 94.4) (width 0.4) (layer "F.Cu") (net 1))
 (segment (start 168.2 112.6) (end 168.2 117.6) (width 0.4) (layer "F.Cu") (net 1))
 (segment (start 173.4 91.6) (end 174.2 90.8) (width 0.4) (layer "F.Cu") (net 1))
 (segment (start 169.435 112.165) (end 169.45 112.15) (width 0.4) (layer "F.Cu") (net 1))
 (segment (start 169 112.6) (end 169.435 112.165) (width 0.4) (layer "F.Cu") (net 1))
 (segment (start 172.7625 108.4) (end 172.395 108.4) (width 0.4) (layer "F.Cu") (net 1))
 (segment (start 180.4 107.8) (end 181.6 107.8) (width 0.4) (layer "F.Cu") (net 1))
 (segment (start 172.6 107.2) (end 172.7625 107.3625) (width 0.4) (layer "F.Cu") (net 1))
 (segment (start 181.6 107.8) (end 182.8 107.8) (width 0.4) (layer "F.Cu") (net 1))
 (segment (start 175.85 100.5125) (end 175.7625 100.6) (width 0.4) (layer "F.Cu") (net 1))
 (segment (start 168.2 112.6) (end 169 112.6) (width 0.4) (layer "F.Cu") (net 1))
 (segment (start 182.8 107.8) (end 183.4 107.2) (width 0.4) (layer "F.Cu") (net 1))
 (segment (start 172.8875 113.0875) (end 172.45 112.65) (width 0.4) (layer "F.Cu") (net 1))
 (segment (start 181.6 101.6) (end 181.6 100.14) (width 0.4) (layer "F.Cu") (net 1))
 (segment (start 186.2 108.2) (end 185.2 107.2) (width 0.4) (layer "F.Cu") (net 1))
 (segment (start 172.7625 107.3625) (end 172.7625 108.4) (width 0.4) (layer "F.Cu") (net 1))
 (segment (start 179.8 91.2) (end 179.8 92.4) (width 0.4) (layer "F.Cu") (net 1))
 (segment (start 175.7625 100.6) (end 175.7625 101.5625) (width 0.4) (layer "F.Cu") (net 1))
 (segment (start 166.075 108.075) (end 165 107) (width 0.4) (layer "F.Cu") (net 1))
 (segment (start 166.895 112.295) (end 167.2 112.6) (width 0.4) (layer "F.Cu") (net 1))
 (segment (start 181.6 101.6) (end 182.8 101.6) (width 0.4) (layer "F.Cu") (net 1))
 (segment (start 172.8875 113.8) (end 172.8875 113.0875) (width 0.4) (layer "F.Cu") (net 1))
 (segment (start 175.85 98.8) (end 175.85 100.5125) (width 0.4) (layer "F.Cu") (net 1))
 (segment (start 181.11 109.29) (end 181.6 108.8) (width 0.4) (layer "F.Cu") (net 1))
 (segment (start 185.3 118.2) (end 186.2 117.3) (width 0.4) (layer "F.Cu") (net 1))
 (segment (start 180.8 102.4) (end 181.6 101.6) (width 0.4) (layer "F.Cu") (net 1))
 (segment (start 182.8 101.6) (end 183.4 101) (width 0.4) (layer "F.Cu") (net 1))
 (segment (start 179.2 95) (end 177.8375 95) (width 0.4) (layer "F.Cu") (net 1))
 (segment (start 162.7 105.3) (end 163 105) (width 0.4) (layer "F.Cu") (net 1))
 (segment (start 183.4 102.2) (end 182.8 101.6) (width 0.4) (layer "F.Cu") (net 1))
 (segment (start 168.2 117.6) (end 168.8 118.2) (width 0.4) (layer "F.Cu") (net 1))
 (segment (start 169.2 96) (end 169.2 97.175) (width 0.4) (layer "F.Cu") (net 12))
 (segment (start 168.2 95) (end 169.2 96) (width 0.4) (layer "F.Cu") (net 12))
 (segment (start 164.025 95) (end 168.2 95) (width 0.4) (layer "F.Cu") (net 12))
 (segment (start 174.8 108.3625) (end 174.8375 108.4) (width 0.4) (layer "F.Cu") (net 8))
 (segment (start 173.8 109.4375) (end 174.8375 108.4) (width 0.4) (layer "F.Cu") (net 8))
 (segment (start 174.8 106.4) (end 174.8 108.3625) (width 0.4) (layer "F.Cu") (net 8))
 (segment (start 173.4 111.2) (end 173.8 110.8) (width 0.4) (layer "F.Cu") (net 8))
 (segment (start 172.45 111.2) (end 173.4 111.2) (width 0.4) (layer "F.Cu") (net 8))
 (segment (start 173.8 110.8) (end 173.8 109.4375) (width 0.4) (layer "F.Cu") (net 8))
 (segment (start 169.435 100.235) (end 169.2 100) (width 0.4) (layer "F.Cu") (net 10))
 (segment (start 169.435 103.125) (end 169.435 100.235) (width 0.4) (layer "F.Cu") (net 10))
 (segment (start 169.2 100) (end 169.2 99) (width 0.4) (layer "F.Cu") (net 10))
 (segment (start 173.8 111.648528) (end 174.248528 111.2) (width 0.4) (layer "F.Cu") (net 6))
 (segment (start 174.248528 111.2) (end 175.15 111.2) (width 0.4) (layer "F.Cu") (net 6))
 (segment (start 173.8 112.8875) (end 173.8 111.648528) (width 0.4) (layer "F.Cu") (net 6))
 (segment (start 174.7125 113.8) (end 173.8 112.8875) (width 0.4) (layer "F.Cu") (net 6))
 (segment (start 168.165 110.565) (end 168.2 110.6) (width 0.4) (layer "F.Cu") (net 9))
 (segment (start 168.165 108.075) (end 168.165 110.565) (width 0.4) (layer "F.Cu") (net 9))
 (segment (start 172.6 104.3625) (end 174.7625 104.3625) (width 0.4) (layer "F.Cu") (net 4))
 (segment (start 182.6 116.4) (end 182.05 115.85) (width 0.4) (layer "F.Cu") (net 4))
 (segment (start 174.7625 104.3625) (end 174.8 104.4) (width 0.4) (layer "F.Cu") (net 4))
 (segment (start 182.05 115.85) (end 180.4 115.85) (width 0.4) (layer "F.Cu") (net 4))
 (segment (start 174.8 104.4) (end 176.8 104.4) (width 0.4) (layer "F.Cu") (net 4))
 (segment (start 172.6 103.6) (end 172.6 104.3625) (width 0.4) (layer "F.Cu") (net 4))
 (segment (start 172.125 103.125) (end 172.6 103.6) (width 0.4) (layer "F.Cu") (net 4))
 (segment (start 184.6 116.4) (end 182.6 116.4) (width 0.4) (layer "F.Cu") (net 4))
 (segment (start 172.4 94.8625) (end 172.4 102.85) (width 0.4) (layer "F.Cu") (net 4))
 (segment (start 170.705 103.125) (end 172.125 103.125) (width 0.4) (layer "F.Cu") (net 4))
 (segment (start 172.4 102.85) (end 172.125 103.125) (width 0.4) (layer "F.Cu") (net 4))
 (segment (start 176.8 104.4) (end 178.6 104.4) (width 0.4) (layer "F.Cu") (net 4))
 (via (at 178.6 104.4) (size 0.8) (drill 0.4) (layers "F.Cu" "B.Cu") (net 4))
 (segment (start 178.6 104.4) (end 178.6 112.4) (width 0.4) (layer "B.Cu") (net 4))
 (segment (start 178.6 112.4) (end 180.4 114.2) (width 0.4) (layer "B.Cu") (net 4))
 (segment (start 180.4 114.2) (end 180.4 115.85) (width 0.4) (layer "B.Cu") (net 4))
 (segment (start 173.35 96.7375) (end 173.35 97.75) (width 0.4) (layer "F.Cu") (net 3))
 (segment (start 175.7625 94.2375) (end 176.2 93.8) (width 0.4) (layer "F.Cu") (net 3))
 (segment (start 176.2 93.8) (end 176.2 92.4) (width 0.4) (layer "F.Cu") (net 3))
 (segment (start 175.8 96.8) (end 173.4125 96.8) (width 0.4) (layer "F.Cu") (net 3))
 (segment (start 175.7625 96.7625) (end 175.8 96.8) (width 0.4) (layer "F.Cu") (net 3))
 (segment (start 176.8 96.8) (end 175.8 96.8) (width 0.4) (layer "F.Cu") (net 3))
 (segment (start 175.7625 95) (end 175.7625 96.7625) (width 0.4) (layer "F.Cu") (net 3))
 (segment (start 173.8 98.2) (end 173.8 99) (width 0.4) (layer "F.Cu") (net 3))
 (segment (start 173.4125 96.8) (end 173.35 96.7375) (width 0.4) (layer "F.Cu") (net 3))
 (segment (start 175.7625 95) (end 175.7625 94.2375) (width 0.4) (layer "F.Cu") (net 3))
 (segment (start 173.35 97.75) (end 173.8 98.2) (width 0.4) (layer "F.Cu") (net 3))
 (segment (start 177.75 98.8) (end 178.6 98.8) (width 0.4) (layer "F.Cu") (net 2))
 (segment (start 179.8 97.6) (end 181.6 97.6) (width 0.4) (layer "F.Cu") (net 2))
 (segment (start 177.75 100.5125) (end 177.8375 100.6) (width 0.4) (layer "F.Cu") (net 2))
 (segment (start 178.6 98.8) (end 179.8 97.6) (width 0.4) (layer "F.Cu") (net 2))
 (segment (start 177.75 98.8) (end 177.75 100.5125) (width 0.4) (layer "F.Cu") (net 2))
 (segment (start 178.4 114.4) (end 179.2 113.6) (width 0.4) (layer "F.Cu") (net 13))
 (segment (start 180.6 113.6) (end 181.11 113.09) (width 0.4) (layer "F.Cu") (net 13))
 (segment (start 178.4 115.85) (end 178.4 114.4) (width 0.4) (layer "F.Cu") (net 13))
 (segment (start 181.11 113.09) (end 181.11 112.15) (width 0.4) (layer "F.Cu") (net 13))
 (segment (start 174.2 116.4) (end 176.2 116.4) (width 0.4) (layer "F.Cu") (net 13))
 (segment (start 176.2 116.4) (end 176.75 115.85) (width 0.4) (layer "F.Cu") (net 13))
 (segment (start 179.2 113.6) (end 180.6 113.6) (width 0.4) (layer "F.Cu") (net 13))
 (segment (start 176.75 115.85) (end 178.4 115.85) (width 0.4) (layer "F.Cu") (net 13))
 (segment (start 177.69 111.2) (end 181.11 111.2) (width 0.4) (layer "F.Cu") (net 15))
 (segment (start 175.15 110.25) (end 177.69 110.25) (width 0.4) (layer "F.Cu") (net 16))
 (segment (start 177.69 112.15) (end 175.15 112.15) (width 0.4) (layer "F.Cu") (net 17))
 (segment (start 176.8 106.4) (end 178.4 106.4) (width 0.4) (layer "F.Cu") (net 5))
 (segment (start 179.54 105.26) (end 181.6 105.26) (width 0.4) (layer "F.Cu") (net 5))
 (segment (start 176.8 106.4) (end 176.8 108.4) (width 0.4) (layer "F.Cu") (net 5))
 (segment (start 178.4 106.4) (end 179.54 105.26) (width 0.4) (layer "F.Cu") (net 5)))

